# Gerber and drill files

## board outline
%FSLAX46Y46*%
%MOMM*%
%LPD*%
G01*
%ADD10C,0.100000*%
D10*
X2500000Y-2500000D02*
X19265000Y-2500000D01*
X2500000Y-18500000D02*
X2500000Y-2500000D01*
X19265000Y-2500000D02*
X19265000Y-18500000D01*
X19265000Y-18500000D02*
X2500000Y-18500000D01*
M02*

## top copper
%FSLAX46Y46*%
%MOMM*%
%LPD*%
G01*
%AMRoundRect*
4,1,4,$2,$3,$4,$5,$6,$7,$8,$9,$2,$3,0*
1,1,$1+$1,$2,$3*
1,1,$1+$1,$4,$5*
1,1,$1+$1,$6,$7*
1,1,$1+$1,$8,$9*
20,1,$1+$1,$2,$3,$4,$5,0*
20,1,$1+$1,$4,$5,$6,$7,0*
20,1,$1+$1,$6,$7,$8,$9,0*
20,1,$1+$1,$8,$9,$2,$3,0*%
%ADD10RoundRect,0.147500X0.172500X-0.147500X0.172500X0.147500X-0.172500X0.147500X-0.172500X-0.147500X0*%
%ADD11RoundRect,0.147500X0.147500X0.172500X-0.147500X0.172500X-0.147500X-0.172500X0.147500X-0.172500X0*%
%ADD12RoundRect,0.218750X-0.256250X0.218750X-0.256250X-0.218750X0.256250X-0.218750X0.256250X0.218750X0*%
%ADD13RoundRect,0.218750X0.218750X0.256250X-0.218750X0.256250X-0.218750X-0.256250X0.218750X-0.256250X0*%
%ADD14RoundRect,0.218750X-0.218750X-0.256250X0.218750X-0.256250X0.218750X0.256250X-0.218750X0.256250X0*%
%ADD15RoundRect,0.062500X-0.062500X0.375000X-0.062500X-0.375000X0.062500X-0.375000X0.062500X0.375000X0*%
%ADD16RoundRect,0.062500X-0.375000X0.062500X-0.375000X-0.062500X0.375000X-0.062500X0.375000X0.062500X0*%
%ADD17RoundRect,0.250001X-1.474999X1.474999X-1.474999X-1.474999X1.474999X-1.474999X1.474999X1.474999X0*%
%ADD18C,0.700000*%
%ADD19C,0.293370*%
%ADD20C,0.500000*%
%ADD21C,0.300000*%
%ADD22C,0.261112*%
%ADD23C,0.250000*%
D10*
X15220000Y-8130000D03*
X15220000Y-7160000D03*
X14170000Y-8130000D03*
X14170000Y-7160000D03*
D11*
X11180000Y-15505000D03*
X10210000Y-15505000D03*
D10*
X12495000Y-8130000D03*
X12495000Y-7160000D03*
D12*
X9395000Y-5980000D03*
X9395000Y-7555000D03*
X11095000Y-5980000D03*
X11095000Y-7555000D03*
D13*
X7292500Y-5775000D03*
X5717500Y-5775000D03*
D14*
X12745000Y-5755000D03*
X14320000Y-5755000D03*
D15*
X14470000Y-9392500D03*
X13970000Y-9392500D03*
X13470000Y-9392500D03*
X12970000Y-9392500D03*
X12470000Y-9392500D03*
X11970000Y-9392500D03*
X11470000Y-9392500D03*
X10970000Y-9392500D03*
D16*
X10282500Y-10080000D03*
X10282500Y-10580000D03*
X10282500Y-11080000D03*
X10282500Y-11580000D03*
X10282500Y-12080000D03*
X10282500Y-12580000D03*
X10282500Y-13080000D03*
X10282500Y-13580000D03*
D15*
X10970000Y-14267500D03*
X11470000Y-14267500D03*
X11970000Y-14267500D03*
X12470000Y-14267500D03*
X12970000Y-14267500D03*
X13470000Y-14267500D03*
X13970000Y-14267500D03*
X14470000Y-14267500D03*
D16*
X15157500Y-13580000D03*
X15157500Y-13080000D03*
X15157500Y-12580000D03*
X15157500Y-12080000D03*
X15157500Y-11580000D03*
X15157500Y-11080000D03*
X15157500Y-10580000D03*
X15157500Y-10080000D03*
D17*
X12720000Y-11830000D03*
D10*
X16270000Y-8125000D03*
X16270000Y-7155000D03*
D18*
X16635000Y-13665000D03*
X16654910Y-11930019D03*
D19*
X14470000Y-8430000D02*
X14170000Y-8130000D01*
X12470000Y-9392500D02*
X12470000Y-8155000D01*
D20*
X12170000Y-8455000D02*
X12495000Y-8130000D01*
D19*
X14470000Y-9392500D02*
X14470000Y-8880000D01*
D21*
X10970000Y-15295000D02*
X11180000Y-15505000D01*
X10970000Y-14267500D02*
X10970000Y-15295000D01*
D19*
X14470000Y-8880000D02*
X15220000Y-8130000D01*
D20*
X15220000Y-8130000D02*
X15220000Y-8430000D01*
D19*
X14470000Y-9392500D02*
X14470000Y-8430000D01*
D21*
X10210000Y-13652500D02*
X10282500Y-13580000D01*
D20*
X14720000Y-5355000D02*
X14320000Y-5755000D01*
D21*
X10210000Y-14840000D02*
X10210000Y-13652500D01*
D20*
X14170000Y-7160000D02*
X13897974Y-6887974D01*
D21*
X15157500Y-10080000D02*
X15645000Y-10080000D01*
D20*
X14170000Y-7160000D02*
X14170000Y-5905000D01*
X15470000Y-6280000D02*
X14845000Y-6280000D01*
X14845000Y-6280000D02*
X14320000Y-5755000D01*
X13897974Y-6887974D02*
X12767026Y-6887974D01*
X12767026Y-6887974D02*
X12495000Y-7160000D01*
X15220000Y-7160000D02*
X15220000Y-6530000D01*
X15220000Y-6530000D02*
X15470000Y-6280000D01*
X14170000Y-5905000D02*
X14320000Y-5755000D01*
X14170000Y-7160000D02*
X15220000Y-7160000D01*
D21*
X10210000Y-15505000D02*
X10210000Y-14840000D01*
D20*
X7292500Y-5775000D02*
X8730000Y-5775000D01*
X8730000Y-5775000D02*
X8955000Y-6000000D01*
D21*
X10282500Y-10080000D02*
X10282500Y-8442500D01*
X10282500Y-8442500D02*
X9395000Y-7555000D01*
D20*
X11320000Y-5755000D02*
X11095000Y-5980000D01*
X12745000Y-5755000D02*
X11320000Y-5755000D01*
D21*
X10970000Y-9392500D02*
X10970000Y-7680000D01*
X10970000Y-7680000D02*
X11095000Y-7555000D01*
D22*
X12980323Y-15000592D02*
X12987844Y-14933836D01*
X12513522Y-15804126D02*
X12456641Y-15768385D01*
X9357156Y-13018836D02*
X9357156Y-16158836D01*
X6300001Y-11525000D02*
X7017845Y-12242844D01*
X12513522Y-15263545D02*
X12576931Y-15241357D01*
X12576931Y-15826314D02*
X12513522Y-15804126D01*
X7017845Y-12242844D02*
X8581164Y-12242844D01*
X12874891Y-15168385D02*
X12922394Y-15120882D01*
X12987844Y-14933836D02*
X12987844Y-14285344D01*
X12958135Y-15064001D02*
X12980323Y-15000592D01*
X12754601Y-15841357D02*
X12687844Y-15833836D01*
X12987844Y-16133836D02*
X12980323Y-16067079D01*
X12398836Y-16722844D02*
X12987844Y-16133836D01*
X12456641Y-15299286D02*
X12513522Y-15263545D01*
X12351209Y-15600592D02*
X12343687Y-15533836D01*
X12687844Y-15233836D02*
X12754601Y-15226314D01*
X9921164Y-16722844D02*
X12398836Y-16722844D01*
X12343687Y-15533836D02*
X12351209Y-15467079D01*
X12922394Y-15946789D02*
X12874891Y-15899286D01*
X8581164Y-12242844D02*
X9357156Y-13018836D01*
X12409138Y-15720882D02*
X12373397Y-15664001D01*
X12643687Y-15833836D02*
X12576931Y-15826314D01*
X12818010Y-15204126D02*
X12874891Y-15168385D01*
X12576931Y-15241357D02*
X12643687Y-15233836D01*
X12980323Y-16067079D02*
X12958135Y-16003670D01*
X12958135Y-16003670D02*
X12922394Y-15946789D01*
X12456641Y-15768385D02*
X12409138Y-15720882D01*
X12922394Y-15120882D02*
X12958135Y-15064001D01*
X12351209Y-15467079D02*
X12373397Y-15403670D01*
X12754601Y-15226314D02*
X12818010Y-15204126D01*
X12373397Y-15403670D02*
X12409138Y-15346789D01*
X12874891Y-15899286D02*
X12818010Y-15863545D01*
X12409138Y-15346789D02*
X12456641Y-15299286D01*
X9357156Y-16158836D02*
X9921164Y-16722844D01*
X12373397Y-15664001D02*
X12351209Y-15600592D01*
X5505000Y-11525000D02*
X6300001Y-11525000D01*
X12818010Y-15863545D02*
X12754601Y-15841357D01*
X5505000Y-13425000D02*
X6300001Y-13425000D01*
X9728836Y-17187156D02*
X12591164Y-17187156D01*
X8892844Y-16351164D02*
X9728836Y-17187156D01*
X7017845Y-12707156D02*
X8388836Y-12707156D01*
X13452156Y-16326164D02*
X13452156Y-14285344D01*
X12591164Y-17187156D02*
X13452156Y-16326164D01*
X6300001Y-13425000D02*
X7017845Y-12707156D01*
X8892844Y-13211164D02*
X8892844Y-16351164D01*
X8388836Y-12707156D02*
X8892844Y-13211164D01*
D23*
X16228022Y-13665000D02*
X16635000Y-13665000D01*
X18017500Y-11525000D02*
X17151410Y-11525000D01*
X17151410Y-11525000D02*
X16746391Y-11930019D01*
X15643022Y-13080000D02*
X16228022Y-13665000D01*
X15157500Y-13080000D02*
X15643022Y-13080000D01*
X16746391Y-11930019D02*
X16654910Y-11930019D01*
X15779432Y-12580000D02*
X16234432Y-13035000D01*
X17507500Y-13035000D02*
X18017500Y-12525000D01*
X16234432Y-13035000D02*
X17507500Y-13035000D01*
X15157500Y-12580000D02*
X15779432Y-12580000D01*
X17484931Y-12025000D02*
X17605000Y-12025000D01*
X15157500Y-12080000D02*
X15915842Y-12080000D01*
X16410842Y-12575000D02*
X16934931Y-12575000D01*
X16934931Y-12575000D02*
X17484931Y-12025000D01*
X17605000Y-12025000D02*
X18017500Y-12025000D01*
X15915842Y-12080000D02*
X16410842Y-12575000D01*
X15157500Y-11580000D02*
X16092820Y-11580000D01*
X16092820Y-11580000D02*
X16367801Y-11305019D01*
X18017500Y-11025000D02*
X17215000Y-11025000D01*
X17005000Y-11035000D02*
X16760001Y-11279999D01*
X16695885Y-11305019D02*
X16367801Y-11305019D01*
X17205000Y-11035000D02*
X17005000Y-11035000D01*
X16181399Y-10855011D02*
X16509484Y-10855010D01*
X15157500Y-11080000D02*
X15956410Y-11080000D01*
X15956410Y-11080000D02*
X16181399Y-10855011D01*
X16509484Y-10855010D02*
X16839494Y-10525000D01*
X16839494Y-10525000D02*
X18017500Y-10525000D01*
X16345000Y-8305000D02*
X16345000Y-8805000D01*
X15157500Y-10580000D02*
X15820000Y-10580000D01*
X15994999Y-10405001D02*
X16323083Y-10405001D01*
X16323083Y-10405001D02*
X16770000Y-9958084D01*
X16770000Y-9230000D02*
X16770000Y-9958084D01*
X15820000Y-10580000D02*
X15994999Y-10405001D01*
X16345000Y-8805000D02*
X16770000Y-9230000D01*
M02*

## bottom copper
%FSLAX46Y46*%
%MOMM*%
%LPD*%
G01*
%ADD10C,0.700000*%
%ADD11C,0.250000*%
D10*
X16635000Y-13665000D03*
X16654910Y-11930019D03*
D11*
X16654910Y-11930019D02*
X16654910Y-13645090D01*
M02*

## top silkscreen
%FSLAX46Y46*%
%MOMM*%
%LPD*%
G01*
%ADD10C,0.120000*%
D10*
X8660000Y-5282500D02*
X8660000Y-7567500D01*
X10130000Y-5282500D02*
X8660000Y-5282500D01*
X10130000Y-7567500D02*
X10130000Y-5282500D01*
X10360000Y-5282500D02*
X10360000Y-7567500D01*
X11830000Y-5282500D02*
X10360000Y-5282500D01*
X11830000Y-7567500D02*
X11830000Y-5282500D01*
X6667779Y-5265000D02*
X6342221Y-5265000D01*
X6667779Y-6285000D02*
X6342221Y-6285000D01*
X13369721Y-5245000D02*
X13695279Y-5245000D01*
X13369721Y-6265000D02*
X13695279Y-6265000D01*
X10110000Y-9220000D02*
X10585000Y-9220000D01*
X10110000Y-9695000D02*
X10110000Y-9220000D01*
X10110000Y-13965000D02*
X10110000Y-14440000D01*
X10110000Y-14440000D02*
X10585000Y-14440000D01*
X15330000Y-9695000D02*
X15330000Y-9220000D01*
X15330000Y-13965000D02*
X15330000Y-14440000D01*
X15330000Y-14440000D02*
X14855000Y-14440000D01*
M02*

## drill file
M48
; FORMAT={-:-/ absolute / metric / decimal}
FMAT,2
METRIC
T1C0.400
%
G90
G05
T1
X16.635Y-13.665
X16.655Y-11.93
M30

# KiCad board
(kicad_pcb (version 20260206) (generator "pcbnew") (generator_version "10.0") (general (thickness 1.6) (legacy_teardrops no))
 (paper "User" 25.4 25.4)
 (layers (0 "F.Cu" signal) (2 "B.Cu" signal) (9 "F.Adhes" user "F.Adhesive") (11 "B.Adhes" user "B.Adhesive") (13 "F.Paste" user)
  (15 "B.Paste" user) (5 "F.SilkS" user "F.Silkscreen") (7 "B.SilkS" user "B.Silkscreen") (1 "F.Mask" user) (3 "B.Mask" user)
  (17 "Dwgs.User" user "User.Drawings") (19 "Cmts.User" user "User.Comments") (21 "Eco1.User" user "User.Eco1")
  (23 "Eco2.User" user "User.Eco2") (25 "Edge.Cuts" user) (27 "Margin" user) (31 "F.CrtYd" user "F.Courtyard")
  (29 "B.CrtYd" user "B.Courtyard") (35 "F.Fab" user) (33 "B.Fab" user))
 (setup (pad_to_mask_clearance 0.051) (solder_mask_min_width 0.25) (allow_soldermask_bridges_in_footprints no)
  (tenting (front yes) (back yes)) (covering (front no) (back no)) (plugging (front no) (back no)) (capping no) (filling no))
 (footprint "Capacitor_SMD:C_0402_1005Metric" (layer "F.Cu") (at 15.22 7.645 90)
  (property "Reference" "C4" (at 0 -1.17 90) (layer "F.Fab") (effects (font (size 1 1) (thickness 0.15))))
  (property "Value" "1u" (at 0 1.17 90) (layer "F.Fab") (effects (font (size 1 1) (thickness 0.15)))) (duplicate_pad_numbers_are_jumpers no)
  (pad "1" smd roundrect (at -0.485 0 90) (size 0.59 0.64) (layers "F.Cu" "F.Mask" "F.Paste") (roundrect_rratio 0.25) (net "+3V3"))
  (pad "2" smd roundrect (at 0.485 0 90) (size 0.59 0.64) (layers "F.Cu" "F.Mask" "F.Paste") (roundrect_rratio 0.25) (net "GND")))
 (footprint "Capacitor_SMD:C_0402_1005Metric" (layer "F.Cu") (at 14.17 7.645 90)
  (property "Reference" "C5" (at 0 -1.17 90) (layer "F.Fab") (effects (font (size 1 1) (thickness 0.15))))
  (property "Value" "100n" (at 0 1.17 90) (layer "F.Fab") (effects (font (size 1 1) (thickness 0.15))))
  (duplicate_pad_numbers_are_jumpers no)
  (pad "1" smd roundrect (at -0.485 0 90) (size 0.59 0.64) (layers "F.Cu" "F.Mask" "F.Paste") (roundrect_rratio 0.25) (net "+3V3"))
  (pad "2" smd roundrect (at 0.485 0 90) (size 0.59 0.64) (layers "F.Cu" "F.Mask" "F.Paste") (roundrect_rratio 0.25) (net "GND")))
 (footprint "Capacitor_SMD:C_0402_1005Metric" (layer "F.Cu") (at 10.695 15.505 180)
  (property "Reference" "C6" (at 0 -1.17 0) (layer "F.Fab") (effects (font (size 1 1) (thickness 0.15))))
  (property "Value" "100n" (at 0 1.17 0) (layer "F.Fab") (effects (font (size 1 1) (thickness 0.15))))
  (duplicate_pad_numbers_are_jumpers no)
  (pad "1" smd roundrect (at -0.485 0 180) (size 0.59 0.64) (layers "F.Cu" "F.Mask" "F.Paste") (roundrect_rratio 0.25) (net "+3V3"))
  (pad "2" smd roundrect (at 0.485 0 180) (size 0.59 0.64) (layers "F.Cu" "F.Mask" "F.Paste") (roundrect_rratio 0.25) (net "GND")))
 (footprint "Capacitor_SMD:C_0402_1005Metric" (layer "F.Cu") (at 12.495 7.645 90)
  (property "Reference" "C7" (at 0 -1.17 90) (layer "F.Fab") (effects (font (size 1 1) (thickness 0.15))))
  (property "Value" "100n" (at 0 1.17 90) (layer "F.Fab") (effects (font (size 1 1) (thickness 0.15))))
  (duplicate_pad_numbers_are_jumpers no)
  (pad "1" smd roundrect (at -0.485 0 90) (size 0.59 0.64) (layers "F.Cu" "F.Mask" "F.Paste") (roundrect_rratio 0.25) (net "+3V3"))
  (pad "2" smd roundrect (at 0.485 0 90) (size 0.59 0.64) (layers "F.Cu" "F.Mask" "F.Paste") (roundrect_rratio 0.25) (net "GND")))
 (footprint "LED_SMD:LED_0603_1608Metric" (layer "F.Cu") (at 9.395 6.7675 -90)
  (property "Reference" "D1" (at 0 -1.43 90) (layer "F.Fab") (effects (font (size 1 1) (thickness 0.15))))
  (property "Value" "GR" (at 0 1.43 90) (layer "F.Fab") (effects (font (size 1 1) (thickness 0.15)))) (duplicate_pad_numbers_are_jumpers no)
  (fp_line (start -1.485 0.735) (end 0.8 0.735) (stroke (width 0.12) (type solid)) (layer "F.SilkS"))
  (fp_line (start -1.485 -0.735) (end -1.485 0.735) (stroke (width 0.12) (type solid)) (layer "F.SilkS"))
  (fp_line (start 0.8 -0.735) (end -1.485 -0.735) (stroke (width 0.12) (type solid)) (layer "F.SilkS"))
  (pad "1" smd roundrect (at -0.7875 0 270) (size 0.875 0.95) (layers "F.Cu" "F.Mask" "F.Paste") (roundrect_rratio 0.25)
   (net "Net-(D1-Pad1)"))
  (pad "2" smd roundrect (at 0.7875 0 270) (size 0.875 0.95) (layers "F.Cu" "F.Mask" "F.Paste") (roundrect_rratio 0.25)
   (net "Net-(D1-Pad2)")))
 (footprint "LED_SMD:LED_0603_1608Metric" (layer "F.Cu") (at 11.095 6.7675 -90)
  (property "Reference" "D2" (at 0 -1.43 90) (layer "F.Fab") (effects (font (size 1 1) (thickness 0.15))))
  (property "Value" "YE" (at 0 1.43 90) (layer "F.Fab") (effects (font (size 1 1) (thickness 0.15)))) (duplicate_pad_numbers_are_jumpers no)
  (fp_line (start -1.485 0.735) (end 0.8 0.735) (stroke (width 0.12) (type solid)) (layer "F.SilkS"))
  (fp_line (start -1.485 -0.735) (end -1.485 0.735) (stroke (width 0.12) (type solid)) (layer "F.SilkS"))
  (fp_line (start 0.8 -0.735) (end -1.485 -0.735) (stroke (width 0.12) (type solid)) (layer "F.SilkS"))
  (pad "1" smd roundrect (at -0.7875 0 270) (size 0.875 0.95) (layers "F.Cu" "F.Mask" "F.Paste") (roundrect_rratio 0.25)
   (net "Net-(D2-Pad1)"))
  (pad "2" smd roundrect (at 0.7875 0 270) (size 0.875 0.95) (layers "F.Cu" "F.Mask" "F.Paste") (roundrect_rratio 0.25)
   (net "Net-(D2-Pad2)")))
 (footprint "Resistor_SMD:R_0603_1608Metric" (layer "F.Cu") (at 6.505 5.775 180)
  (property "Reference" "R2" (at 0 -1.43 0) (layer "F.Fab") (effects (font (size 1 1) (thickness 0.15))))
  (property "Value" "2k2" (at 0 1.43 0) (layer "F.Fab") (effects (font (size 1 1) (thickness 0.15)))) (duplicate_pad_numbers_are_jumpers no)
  (fp_line (start -0.162779 0.51) (end 0.162779 0.51) (stroke (width 0.12) (type solid)) (layer "F.SilkS"))
  (fp_line (start -0.162779 -0.51) (end 0.162779 -0.51) (stroke (width 0.12) (type solid)) (layer "F.SilkS"))
  (pad "1" smd roundrect (at -0.7875 0 180) (size 0.875 0.95) (layers "F.Cu" "F.Mask" "F.Paste") (roundrect_rratio 0.25)
   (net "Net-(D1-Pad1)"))
  (pad "2" smd roundrect (at 0.7875 0 180) (size 0.875 0.95) (layers "F.Cu" "F.Mask" "F.Paste") (roundrect_rratio 0.25) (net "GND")))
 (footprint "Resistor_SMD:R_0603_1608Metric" (layer "F.Cu") (at 13.5325 5.755)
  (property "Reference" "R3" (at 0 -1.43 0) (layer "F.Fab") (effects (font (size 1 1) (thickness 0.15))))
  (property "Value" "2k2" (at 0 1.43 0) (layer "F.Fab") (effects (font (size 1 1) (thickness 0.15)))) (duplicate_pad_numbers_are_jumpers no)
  (fp_line (start -0.162779 -0.51) (end 0.162779 -0.51) (stroke (width 0.12) (type solid)) (layer "F.SilkS"))
  (fp_line (start -0.162779 0.51) (end 0.162779 0.51) (stroke (width 0.12) (type solid)) (layer "F.SilkS"))
  (pad "1" smd roundrect (at -0.7875 0) (size 0.875 0.95) (layers "F.Cu" "F.Mask" "F.Paste") (roundrect_rratio 0.25) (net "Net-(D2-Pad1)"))
  (pad "2" smd roundrect (at 0.7875 0) (size 0.875 0.95) (layers "F.Cu" "F.Mask" "F.Paste") (roundrect_rratio 0.25) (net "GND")))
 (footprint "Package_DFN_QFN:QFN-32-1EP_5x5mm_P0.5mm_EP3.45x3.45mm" (layer "F.Cu") (at 12.72 11.83 -90)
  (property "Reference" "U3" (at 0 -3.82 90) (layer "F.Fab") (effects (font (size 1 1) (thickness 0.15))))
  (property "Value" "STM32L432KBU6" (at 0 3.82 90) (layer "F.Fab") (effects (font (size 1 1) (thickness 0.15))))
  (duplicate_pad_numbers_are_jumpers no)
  (fp_line (start -2.61 2.61) (end -2.61 2.135) (stroke (width 0.12) (type solid)) (layer "F.SilkS"))
  (fp_line (start -2.135 2.61) (end -2.61 2.61) (stroke (width 0.12) (type solid)) (layer "F.SilkS"))
  (fp_line (start 2.135 2.61) (end 2.61 2.61) (stroke (width 0.12) (type solid)) (layer "F.SilkS"))
  (fp_line (start 2.61 2.61) (end 2.61 2.135) (stroke (width 0.12) (type solid)) (layer "F.SilkS"))
  (fp_line (start -2.135 -2.61) (end -2.61 -2.61) (stroke (width 0.12) (type solid)) (layer "F.SilkS"))
  (fp_line (start 2.135 -2.61) (end 2.61 -2.61) (stroke (width 0.12) (type solid)) (layer "F.SilkS"))
  (fp_line (start 2.61 -2.61) (end 2.61 -2.135) (stroke (width 0.12) (type solid)) (layer "F.SilkS"))
  (pad "" smd roundrect (at -1.15 -1.15 270) (size 0.93 0.93) (layers "F.Paste") (roundrect_rratio 0.25))
  (pad "" smd roundrect (at -1.15 0 270) (size 0.93 0.93) (layers "F.Paste") (roundrect_rratio 0.25))
  (pad "" smd roundrect (at -1.15 1.15 270) (size 0.93 0.93) (layers "F.Paste") (roundrect_rratio 0.25))
  (pad "" smd roundrect (at 0 -1.15 270) (size 0.93 0.93) (layers "F.Paste") (roundrect_rratio 0.25))
  (pad "" smd roundrect (at 0 0 270) (size 0.93 0.93) (layers "F.Paste") (roundrect_rratio 0.25))
  (pad "" smd roundrect (at 0 1.15 270) (size 0.93 0.93) (layers "F.Paste") (roundrect_rratio 0.25))
  (pad "" smd roundrect (at 1.15 -1.15 270) (size 0.93 0.93) (layers "F.Paste") (roundrect_rratio 0.25))
  (pad "" smd roundrect (at 1.15 0 270) (size 0.93 0.93) (layers "F.Paste") (roundrect_rratio 0.25))
  (pad "" smd roundrect (at 1.15 1.15 270) (size 0.93 0.93) (layers "F.Paste") (roundrect_rratio 0.25))
  (pad "1" smd roundrect (at -2.4375 -1.75 270) (size 0.875 0.25) (layers "F.Cu" "F.Mask" "F.Paste") (roundrect_rratio 0.25) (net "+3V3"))
  (pad "2" smd roundrect (at -2.4375 -1.25 270) (size 0.875 0.25) (layers "F.Cu" "F.Mask" "F.Paste") (roundrect_rratio 0.25)
   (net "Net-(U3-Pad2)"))
  (pad "3" smd roundrect (at -2.4375 -0.75 270) (size 0.875 0.25) (layers "F.Cu" "F.Mask" "F.Paste") (roundrect_rratio 0.25)
   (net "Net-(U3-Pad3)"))
  (pad "4" smd roundrect (at -2.4375 -0.25 270) (size 0.875 0.25) (layers "F.Cu" "F.Mask" "F.Paste") (roundrect_rratio 0.25) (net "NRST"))
  (pad "5" smd roundrect (at -2.4375 0.25 270) (size 0.875 0.25) (layers "F.Cu" "F.Mask" "F.Paste") (roundrect_rratio 0.25) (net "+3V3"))
  (pad "6" smd roundrect (at -2.4375 0.75 270) (size 0.875 0.25) (layers "F.Cu" "F.Mask" "F.Paste") (roundrect_rratio 0.25)
   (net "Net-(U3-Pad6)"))
  (pad "7" smd roundrect (at -2.4375 1.25 270) (size 0.875 0.25) (layers "F.Cu" "F.Mask" "F.Paste") (roundrect_rratio 0.25)
   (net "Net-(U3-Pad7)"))
  (pad "8" smd roundrect (at -2.4375 1.75 270) (size 0.875 0.25) (layers "F.Cu" "F.Mask" "F.Paste") (roundrect_rratio 0.25)
   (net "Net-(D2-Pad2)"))
  (pad "9" smd roundrect (at -1.75 2.4375 270) (size 0.25 0.875) (layers "F.Cu" "F.Mask" "F.Paste") (roundrect_rratio 0.25)
   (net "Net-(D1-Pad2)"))
  (pad "10" smd roundrect (at -1.25 2.4375 270) (size 0.25 0.875) (layers "F.Cu" "F.Mask" "F.Paste") (roundrect_rratio 0.25)
   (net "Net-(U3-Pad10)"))
  (pad "11" smd roundrect (at -0.75 2.4375 270) (size 0.25 0.875) (layers "F.Cu" "F.Mask" "F.Paste") (roundrect_rratio 0.25)
   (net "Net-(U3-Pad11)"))
  (pad "12" smd roundrect (at -0.25 2.4375 270) (size 0.25 0.875) (layers "F.Cu" "F.Mask" "F.Paste") (roundrect_rratio 0.25)
   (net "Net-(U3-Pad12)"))
  (pad "13" smd roundrect (at 0.25 2.4375 270) (size 0.25 0.875) (layers "F.Cu" "F.Mask" "F.Paste") (roundrect_rratio 0.25)
   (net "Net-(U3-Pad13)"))
  (pad "14" smd roundrect (at 0.75 2.4375 270) (size 0.25 0.875) (layers "F.Cu" "F.Mask" "F.Paste") (roundrect_rratio 0.25)
   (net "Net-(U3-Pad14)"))
  (pad "15" smd roundrect (at 1.25 2.4375 270) (size 0.25 0.875) (layers "F.Cu" "F.Mask" "F.Paste") (roundrect_rratio 0.25)
   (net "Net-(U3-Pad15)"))
  (pad "16" smd roundrect (at 1.75 2.4375 270) (size 0.25 0.875) (layers "F.Cu" "F.Mask" "F.Paste") (roundrect_rratio 0.25) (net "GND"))
  (pad "17" smd roundrect (at 2.4375 1.75 270) (size 0.875 0.25) (layers "F.Cu" "F.Mask" "F.Paste") (roundrect_rratio 0.25) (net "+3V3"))
  (pad "18" smd roundrect (at 2.4375 1.25 270) (size 0.875 0.25) (layers "F.Cu" "F.Mask" "F.Paste") (roundrect_rratio 0.25)
   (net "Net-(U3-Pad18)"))
  (pad "19" smd roundrect (at 2.4375 0.75 270) (size 0.875 0.25) (layers "F.Cu" "F.Mask" "F.Paste") (roundrect_rratio 0.25)
   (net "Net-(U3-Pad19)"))
  (pad "20" smd roundrect (at 2.4375 0.25 270) (size 0.875 0.25) (layers "F.Cu" "F.Mask" "F.Paste") (roundrect_rratio 0.25)
   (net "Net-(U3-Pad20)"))
  (pad "21" smd roundrect (at 2.4375 -0.25 270) (size 0.875 0.25) (layers "F.Cu" "F.Mask" "F.Paste") (roundrect_rratio 0.25) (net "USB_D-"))
  (pad "22" smd roundrect (at 2.4375 -0.75 270) (size 0.875 0.25) (layers "F.Cu" "F.Mask" "F.Paste") (roundrect_rratio 0.25) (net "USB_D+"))
  (pad "23" smd roundrect (at 2.4375 -1.25 270) (size 0.875 0.25) (layers "F.Cu" "F.Mask" "F.Paste") (roundrect_rratio 0.25) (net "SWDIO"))
  (pad "24" smd roundrect (at 2.4375 -1.75 270) (size 0.875 0.25) (layers "F.Cu" "F.Mask" "F.Paste") (roundrect_rratio 0.25) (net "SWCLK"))
  (pad "25" smd roundrect (at 1.75 -2.4375 270) (size 0.25 0.875) (layers "F.Cu" "F.Mask" "F.Paste") (roundrect_rratio 0.25) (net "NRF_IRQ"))
  (pad "26" smd roundrect (at 1.25 -2.4375 270) (size 0.25 0.875) (layers "F.Cu" "F.Mask" "F.Paste") (roundrect_rratio 0.25)
   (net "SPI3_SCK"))
  (pad "27" smd roundrect (at 0.75 -2.4375 270) (size 0.25 0.875) (layers "F.Cu" "F.Mask" "F.Paste") (roundrect_rratio 0.25)
   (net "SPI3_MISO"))
  (pad "28" smd roundrect (at 0.25 -2.4375 270) (size 0.25 0.875) (layers "F.Cu" "F.Mask" "F.Paste") (roundrect_rratio 0.25)
   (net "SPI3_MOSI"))
  (pad "29" smd roundrect (at -0.25 -2.4375 270) (size 0.25 0.875) (layers "F.Cu" "F.Mask" "F.Paste") (roundrect_rratio 0.25)
   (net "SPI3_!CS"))
  (pad "30" smd roundrect (at -0.75 -2.4375 270) (size 0.25 0.875) (layers "F.Cu" "F.Mask" "F.Paste") (roundrect_rratio 0.25) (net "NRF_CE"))
  (pad "31" smd roundrect (at -1.25 -2.4375 270) (size 0.25 0.875) (layers "F.Cu" "F.Mask" "F.Paste") (roundrect_rratio 0.25)
   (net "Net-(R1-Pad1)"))
  (pad "32" smd roundrect (at -1.75 -2.4375 270) (size 0.25 0.875) (layers "F.Cu" "F.Mask" "F.Paste") (roundrect_rratio 0.25) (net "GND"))
  (pad "33" smd roundrect (at 0 0 270) (size 3.45 3.45) (layers "F.Cu" "F.Mask") (roundrect_rratio 0.072464) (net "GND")))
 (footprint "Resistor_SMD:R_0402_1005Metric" (layer "F.Cu") (at 16.27 7.64 90)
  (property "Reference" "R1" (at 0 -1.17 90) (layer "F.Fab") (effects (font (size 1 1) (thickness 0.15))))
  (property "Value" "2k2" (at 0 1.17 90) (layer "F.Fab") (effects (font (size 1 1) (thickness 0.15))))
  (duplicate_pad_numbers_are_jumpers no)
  (pad "1" smd roundrect (at -0.485 0 90) (size 0.59 0.64) (layers "F.Cu" "F.Mask" "F.Paste") (roundrect_rratio 0.25) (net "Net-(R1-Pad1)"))
  (pad "2" smd roundrect (at 0.485 0 90) (size 0.59 0.64) (layers "F.Cu" "F.Mask" "F.Paste") (roundrect_rratio 0.25) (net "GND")))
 (gr_line (start 2.5 2.5) (end 19.265 2.5) (stroke (width 0.1) (type default)) (layer "Edge.Cuts"))
 (gr_line (start 2.5 18.5) (end 2.5 2.5) (stroke (width 0.1) (type default)) (layer "Edge.Cuts"))
 (gr_line (start 19.265 2.5) (end 19.265 18.5) (stroke (width 0.1) (type default)) (layer "Edge.Cuts"))
 (gr_line (start 19.265 18.5) (end 2.5 18.5) (stroke (width 0.1) (type default)) (layer "Edge.Cuts"))
 (segment (start 14.47 8.43) (end 14.17 8.13) (width 0.29337) (layer "F.Cu") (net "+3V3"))
 (segment (start 12.47 9.3925) (end 12.47 8.155) (width 0.29337) (layer "F.Cu") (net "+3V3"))
 (segment (start 12.17 8.455) (end 12.495 8.13) (width 0.5) (layer "F.Cu") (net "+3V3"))
 (segment (start 14.47 9.3925) (end 14.47 8.88) (width 0.29337) (layer "F.Cu") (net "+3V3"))
 (segment (start 10.97 15.295) (end 11.18 15.505) (width 0.3) (layer "F.Cu") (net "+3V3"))
 (segment (start 10.97 14.2675) (end 10.97 15.295) (width 0.3) (layer "F.Cu") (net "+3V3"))
 (segment (start 14.47 8.88) (end 15.22 8.13) (width 0.29337) (layer "F.Cu") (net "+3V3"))
 (segment (start 15.22 8.13) (end 15.22 8.43) (width 0.5) (layer "F.Cu") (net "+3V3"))
 (segment (start 14.47 9.3925) (end 14.47 8.43) (width 0.29337) (layer "F.Cu") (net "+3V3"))
 (segment (start 10.21 13.6525) (end 10.2825 13.58) (width 0.3) (layer "F.Cu") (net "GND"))
 (segment (start 14.72 5.355) (end 14.32 5.755) (width 0.5) (layer "F.Cu") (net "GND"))
 (segment (start 10.21 14.84) (end 10.21 13.6525) (width 0.3) (layer "F.Cu") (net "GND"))
 (segment (start 14.17 7.16) (end 13.897974 6.887974) (width 0.5) (layer "F.Cu") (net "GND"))
 (segment (start 15.1575 10.08) (end 15.645 10.08) (width 0.3) (layer "F.Cu") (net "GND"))
 (segment (start 14.17 7.16) (end 14.17 5.905) (width 0.5) (layer "F.Cu") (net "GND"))
 (segment (start 15.47 6.28) (end 14.845 6.28) (width 0.5) (layer "F.Cu") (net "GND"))
 (segment (start 14.845 6.28) (end 14.32 5.755) (width 0.5) (layer "F.Cu") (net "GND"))
 (segment (start 13.897974 6.887974) (end 12.767026 6.887974) (width 0.5) (layer "F.Cu") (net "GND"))
 (segment (start 12.767026 6.887974) (end 12.495 7.16) (width 0.5) (layer "F.Cu") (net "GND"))
 (segment (start 15.22 7.16) (end 15.22 6.53) (width 0.5) (layer "F.Cu") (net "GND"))
 (segment (start 15.22 6.53) (end 15.47 6.28) (width 0.5) (layer "F.Cu") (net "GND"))
 (segment (start 14.17 5.905) (end 14.32 5.755) (width 0.5) (layer "F.Cu") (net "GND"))
 (segment (start 14.17 7.16) (end 15.22 7.16) (width 0.5) (layer "F.Cu") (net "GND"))
 (segment (start 10.21 15.505) (end 10.21 14.84) (width 0.3) (layer "F.Cu") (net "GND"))
 (segment (start 7.2925 5.775) (end 8.73 5.775) (width 0.5) (layer "F.Cu") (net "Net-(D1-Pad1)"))
 (segment (start 8.73 5.775) (end 8.955 6) (width 0.5) (layer "F.Cu") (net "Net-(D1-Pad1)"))
 (segment (start 10.2825 10.08) (end 10.2825 8.4425) (width 0.3) (layer "F.Cu") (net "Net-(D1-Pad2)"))
 (segment (start 10.2825 8.4425) (end 9.395 7.555) (width 0.3) (layer "F.Cu") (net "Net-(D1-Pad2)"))
 (segment (start 11.32 5.755) (end 11.095 5.98) (width 0.5) (layer "F.Cu") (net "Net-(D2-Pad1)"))
 (segment (start 12.745 5.755) (end 11.32 5.755) (width 0.5) (layer "F.Cu") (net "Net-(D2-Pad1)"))
 (segment (start 10.97 9.3925) (end 10.97 7.68) (width 0.3) (layer "F.Cu") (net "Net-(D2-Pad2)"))
 (segment (start 10.97 7.68) (end 11.095 7.555) (width 0.3) (layer "F.Cu") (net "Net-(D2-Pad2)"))
 (segment (start 12.980323 15.000592) (end 12.987844 14.933836) (width 0.261112) (layer "F.Cu") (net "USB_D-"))
 (segment (start 12.513522 15.804126) (end 12.456641 15.768385) (width 0.261112) (layer "F.Cu") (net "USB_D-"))
 (segment (start 9.357156 13.018836) (end 9.357156 16.158836) (width 0.261112) (layer "F.Cu") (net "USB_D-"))
 (segment (start 6.300001 11.525) (end 7.017845 12.242844) (width 0.261112) (layer "F.Cu") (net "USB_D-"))
 (segment (start 12.513522 15.263545) (end 12.576931 15.241357) (width 0.261112) (layer "F.Cu") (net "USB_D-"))
 (segment (start 12.576931 15.826314) (end 12.513522 15.804126) (width 0.261112) (layer "F.Cu") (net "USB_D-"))
 (segment (start 7.017845 12.242844) (end 8.581164 12.242844) (width 0.261112) (layer "F.Cu") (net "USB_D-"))
 (segment (start 12.874891 15.168385) (end 12.922394 15.120882) (width 0.261112) (layer "F.Cu") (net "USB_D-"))
 (segment (start 12.987844 14.933836) (end 12.987844 14.285344) (width 0.261112) (layer "F.Cu") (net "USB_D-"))
 (segment (start 12.958135 15.064001) (end 12.980323 15.000592) (width 0.261112) (layer "F.Cu") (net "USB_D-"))
 (segment (start 12.754601 15.841357) (end 12.687844 15.833836) (width 0.261112) (layer "F.Cu") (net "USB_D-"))
 (segment (start 12.987844 16.133836) (end 12.980323 16.067079) (width 0.261112) (layer "F.Cu") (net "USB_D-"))
 (segment (start 12.398836 16.722844) (end 12.987844 16.133836) (width 0.261112) (layer "F.Cu") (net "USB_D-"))
 (segment (start 12.456641 15.299286) (end 12.513522 15.263545) (width 0.261112) (layer "F.Cu") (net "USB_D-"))
 (segment (start 12.351209 15.600592) (end 12.343687 15.533836) (width 0.261112) (layer "F.Cu") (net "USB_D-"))
 (segment (start 12.687844 15.233836) (end 12.754601 15.226314) (width 0.261112) (layer "F.Cu") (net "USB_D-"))
 (segment (start 9.921164 16.722844) (end 12.398836 16.722844) (width 0.261112) (layer "F.Cu") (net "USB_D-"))
 (segment (start 12.343687 15.533836) (end 12.351209 15.467079) (width 0.261112) (layer "F.Cu") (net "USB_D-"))
 (segment (start 12.922394 15.946789) (end 12.874891 15.899286) (width 0.261112) (layer "F.Cu") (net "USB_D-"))
 (segment (start 8.581164 12.242844) (end 9.357156 13.018836) (width 0.261112) (layer "F.Cu") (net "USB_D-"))
 (segment (start 12.409138 15.720882) (end 12.373397 15.664001) (width 0.261112) (layer "F.Cu") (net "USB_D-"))
 (segment (start 12.643687 15.833836) (end 12.576931 15.826314) (width 0.261112) (layer "F.Cu") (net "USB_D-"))
 (segment (start 12.81801 15.204126) (end 12.874891 15.168385) (width 0.261112) (layer "F.Cu") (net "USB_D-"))
 (segment (start 12.576931 15.241357) (end 12.643687 15.233836) (width 0.261112) (layer "F.Cu") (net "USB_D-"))
 (segment (start 12.980323 16.067079) (end 12.958135 16.00367) (width 0.261112) (layer "F.Cu") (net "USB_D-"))
 (segment (start 12.958135 16.00367) (end 12.922394 15.946789) (width 0.261112) (layer "F.Cu") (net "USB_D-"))
 (segment (start 12.456641 15.768385) (end 12.409138 15.720882) (width 0.261112) (layer "F.Cu") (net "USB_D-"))
 (segment (start 12.922394 15.120882) (end 12.958135 15.064001) (width 0.261112) (layer "F.Cu") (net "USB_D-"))
 (segment (start 12.351209 15.467079) (end 12.373397 15.40367) (width 0.261112) (layer "F.Cu") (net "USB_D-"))
 (segment (start 12.754601 15.226314) (end 12.81801 15.204126) (width 0.261112) (layer "F.Cu") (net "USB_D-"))
 (segment (start 12.373397 15.40367) (end 12.409138 15.346789) (width 0.261112) (layer "F.Cu") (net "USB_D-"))
 (segment (start 12.874891 15.899286) (end 12.81801 15.863545) (width 0.261112) (layer "F.Cu") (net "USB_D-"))
 (segment (start 12.409138 15.346789) (end 12.456641 15.299286) (width 0.261112) (layer "F.Cu") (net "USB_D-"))
 (segment (start 9.357156 16.158836) (end 9.921164 16.722844) (width 0.261112) (layer "F.Cu") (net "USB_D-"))
 (segment (start 12.373397 15.664001) (end 12.351209 15.600592) (width 0.261112) (layer "F.Cu") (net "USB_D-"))
 (segment (start 5.505 11.525) (end 6.300001 11.525) (width 0.261112) (layer "F.Cu") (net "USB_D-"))
 (segment (start 12.81801 15.863545) (end 12.754601 15.841357) (width 0.261112) (layer "F.Cu") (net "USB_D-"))
 (segment (start 5.505 13.425) (end 6.300001 13.425) (width 0.261112) (layer "F.Cu") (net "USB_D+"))
 (segment (start 9.728836 17.187156) (end 12.591164 17.187156) (width 0.261112) (layer "F.Cu") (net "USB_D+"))
 (segment (start 8.892844 16.351164) (end 9.728836 17.187156) (width 0.261112) (layer "F.Cu") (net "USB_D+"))
 (segment (start 7.017845 12.707156) (end 8.388836 12.707156) (width 0.261112) (layer "F.Cu") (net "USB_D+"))
 (segment (start 13.452156 16.326164) (end 13.452156 14.285344) (width 0.261112) (layer "F.Cu") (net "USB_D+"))
 (segment (start 12.591164 17.187156) (end 13.452156 16.326164) (width 0.261112) (layer "F.Cu") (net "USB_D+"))
 (segment (start 6.300001 13.425) (end 7.017845 12.707156) (width 0.261112) (layer "F.Cu") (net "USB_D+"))
 (segment (start 8.892844 13.211164) (end 8.892844 16.351164) (width 0.261112) (layer "F.Cu") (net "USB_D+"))
 (segment (start 8.388836 12.707156) (end 8.892844 13.211164) (width 0.261112) (layer "F.Cu") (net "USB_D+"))
 (segment (start 16.228022 13.665) (end 16.635 13.665) (width 0.25) (layer "F.Cu") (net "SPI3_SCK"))
 (segment (start 18.0175 11.525) (end 17.15141 11.525) (width 0.25) (layer "F.Cu") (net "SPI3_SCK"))
 (segment (start 17.15141 11.525) (end 16.746391 11.930019) (width 0.25) (layer "F.Cu") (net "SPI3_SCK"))
 (segment (start 15.643022 13.08) (end 16.228022 13.665) (width 0.25) (layer "F.Cu") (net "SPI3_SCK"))
 (segment (start 15.1575 13.08) (end 15.643022 13.08) (width 0.25) (layer "F.Cu") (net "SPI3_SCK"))
 (segment (start 16.746391 11.930019) (end 16.65491 11.930019) (width 0.25) (layer "F.Cu") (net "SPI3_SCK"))
 (via (at 16.635 13.665) (size 0.7) (drill 0.4) (layers "F.Cu" "B.Cu") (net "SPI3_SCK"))
 (via (at 16.65491 11.930019) (size 0.7) (drill 0.4) (layers "F.Cu" "B.Cu") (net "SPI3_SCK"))
 (segment (start 16.65491 11.930019) (end 16.65491 13.64509) (width 0.25) (layer "B.Cu") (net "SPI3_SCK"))
 (segment (start 15.779432 12.58) (end 16.234432 13.035) (width 0.25) (layer "F.Cu") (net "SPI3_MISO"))
 (segment (start 17.5075 13.035) (end 18.0175 12.525) (width 0.25) (layer "F.Cu") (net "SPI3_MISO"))
 (segment (start 16.234432 13.035) (end 17.5075 13.035) (width 0.25) (layer "F.Cu") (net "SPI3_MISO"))
 (segment (start 15.1575 12.58) (end 15.779432 12.58) (width 0.25) (layer "F.Cu") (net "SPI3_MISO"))
 (segment (start 17.484931 12.025) (end 17.605 12.025) (width 0.25) (layer "F.Cu") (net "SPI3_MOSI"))
 (segment (start 15.1575 12.08) (end 15.915842 12.08) (width 0.25) (layer "F.Cu") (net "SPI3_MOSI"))
 (segment (start 16.410842 12.575) (end 16.934931 12.575) (width 0.25) (layer "F.Cu") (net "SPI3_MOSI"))
 (segment (start 16.934931 12.575) (end 17.484931 12.025) (width 0.25) (layer "F.Cu") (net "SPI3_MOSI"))
 (segment (start 17.605 12.025) (end 18.0175 12.025) (width 0.25) (layer "F.Cu") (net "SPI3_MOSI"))
 (segment (start 15.915842 12.08) (end 16.410842 12.575) (width 0.25) (layer "F.Cu") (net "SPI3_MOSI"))
 (segment (start 15.1575 11.58) (end 16.09282 11.58) (width 0.25) (layer "F.Cu") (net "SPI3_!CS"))
 (segment (start 16.09282 11.58) (end 16.367801 11.305019) (width 0.25) (layer "F.Cu") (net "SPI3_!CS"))
 (segment (start 18.0175 11.025) (end 17.215 11.025) (width 0.25) (layer "F.Cu") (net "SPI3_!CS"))
 (segment (start 17.005 11.035) (end 16.760001 11.279999) (width 0.25) (layer "F.Cu") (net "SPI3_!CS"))
 (segment (start 16.695885 11.305019) (end 16.367801 11.305019) (width 0.25) (layer "F.Cu") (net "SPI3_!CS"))
 (segment (start 17.205 11.035) (end 17.005 11.035) (width 0.25) (layer "F.Cu") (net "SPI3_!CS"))
 (segment (start 16.181399 10.855011) (end 16.509484 10.85501) (width 0.25) (layer "F.Cu") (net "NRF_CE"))
 (segment (start 15.1575 11.08) (end 15.95641 11.08) (width 0.25) (layer "F.Cu") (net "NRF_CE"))
 (segment (start 15.95641 11.08) (end 16.181399 10.855011) (width 0.25) (layer "F.Cu") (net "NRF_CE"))
 (segment (start 16.509484 10.85501) (end 16.839494 10.525) (width 0.25) (layer "F.Cu") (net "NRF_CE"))
 (segment (start 16.839494 10.525) (end 18.0175 10.525) (width 0.25) (layer "F.Cu") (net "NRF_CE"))
 (segment (start 16.345 8.305) (end 16.345 8.805) (width 0.25) (layer "F.Cu") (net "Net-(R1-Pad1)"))
 (segment (start 15.1575 10.58) (end 15.82 10.58) (width 0.25) (layer "F.Cu") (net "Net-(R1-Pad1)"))
 (segment (start 15.994999 10.405001) (end 16.323083 10.405001) (width 0.25) (layer "F.Cu") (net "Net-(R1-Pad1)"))
 (segment (start 16.323083 10.405001) (end 16.77 9.958084) (width 0.25) (layer "F.Cu") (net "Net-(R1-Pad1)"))
 (segment (start 16.77 9.23) (end 16.77 9.958084) (width 0.25) (layer "F.Cu") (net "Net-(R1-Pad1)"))
 (segment (start 15.82 10.58) (end 15.994999 10.405001) (width 0.25) (layer "F.Cu") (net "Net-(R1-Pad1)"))
 (segment (start 16.345 8.805) (end 16.77 9.23) (width 0.25) (layer "F.Cu") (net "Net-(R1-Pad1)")))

